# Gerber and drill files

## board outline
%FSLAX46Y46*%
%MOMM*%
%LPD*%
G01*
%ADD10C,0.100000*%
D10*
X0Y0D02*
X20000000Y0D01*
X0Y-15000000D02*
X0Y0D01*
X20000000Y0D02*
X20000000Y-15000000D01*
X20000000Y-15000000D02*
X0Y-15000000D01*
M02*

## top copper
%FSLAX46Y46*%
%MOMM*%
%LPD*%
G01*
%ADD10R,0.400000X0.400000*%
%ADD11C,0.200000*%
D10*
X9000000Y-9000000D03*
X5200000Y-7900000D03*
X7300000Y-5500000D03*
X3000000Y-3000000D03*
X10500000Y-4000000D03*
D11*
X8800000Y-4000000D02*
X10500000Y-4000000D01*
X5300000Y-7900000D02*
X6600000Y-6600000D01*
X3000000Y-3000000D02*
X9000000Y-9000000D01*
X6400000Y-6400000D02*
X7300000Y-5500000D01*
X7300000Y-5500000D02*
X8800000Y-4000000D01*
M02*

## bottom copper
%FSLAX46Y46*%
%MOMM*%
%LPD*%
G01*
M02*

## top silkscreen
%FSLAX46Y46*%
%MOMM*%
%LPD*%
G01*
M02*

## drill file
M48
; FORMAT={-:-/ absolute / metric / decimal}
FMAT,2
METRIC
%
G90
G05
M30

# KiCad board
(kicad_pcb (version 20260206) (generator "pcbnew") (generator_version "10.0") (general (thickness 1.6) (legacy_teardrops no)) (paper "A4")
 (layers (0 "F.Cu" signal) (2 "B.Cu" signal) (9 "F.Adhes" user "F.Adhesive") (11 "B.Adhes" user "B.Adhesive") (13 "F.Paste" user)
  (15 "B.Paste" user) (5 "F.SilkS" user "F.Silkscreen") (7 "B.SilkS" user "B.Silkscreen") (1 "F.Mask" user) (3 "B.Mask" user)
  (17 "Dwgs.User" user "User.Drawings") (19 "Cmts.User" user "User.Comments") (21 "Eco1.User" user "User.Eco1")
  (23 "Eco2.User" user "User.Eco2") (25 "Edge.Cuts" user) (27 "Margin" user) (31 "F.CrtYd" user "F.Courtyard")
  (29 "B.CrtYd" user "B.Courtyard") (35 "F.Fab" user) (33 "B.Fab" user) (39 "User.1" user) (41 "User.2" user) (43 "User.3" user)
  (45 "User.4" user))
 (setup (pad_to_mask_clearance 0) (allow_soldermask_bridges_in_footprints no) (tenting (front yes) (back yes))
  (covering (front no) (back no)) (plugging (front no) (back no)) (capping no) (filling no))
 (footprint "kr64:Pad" (layer "F.Cu") (at 9 9)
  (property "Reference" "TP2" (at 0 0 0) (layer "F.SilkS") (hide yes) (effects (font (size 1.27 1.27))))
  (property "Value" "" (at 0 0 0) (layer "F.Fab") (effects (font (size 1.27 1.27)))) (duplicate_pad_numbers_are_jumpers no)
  (pad "1" smd rect (at 0 0) (size 0.4 0.4) (layers "F.Cu" "F.Mask" "F.Paste") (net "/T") (thermal_bridge_angle 45)))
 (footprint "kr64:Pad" (layer "F.Cu") (at 5.2 7.9)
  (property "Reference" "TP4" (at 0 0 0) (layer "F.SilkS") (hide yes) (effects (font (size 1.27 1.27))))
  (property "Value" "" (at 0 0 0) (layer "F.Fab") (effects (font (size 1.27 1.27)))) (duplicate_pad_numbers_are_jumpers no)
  (pad "1" smd rect (at 0 0) (size 0.4 0.4) (layers "F.Cu" "F.Mask" "F.Paste") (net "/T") (thermal_bridge_angle 45)))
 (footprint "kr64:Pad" (layer "F.Cu") (at 7.3 5.5)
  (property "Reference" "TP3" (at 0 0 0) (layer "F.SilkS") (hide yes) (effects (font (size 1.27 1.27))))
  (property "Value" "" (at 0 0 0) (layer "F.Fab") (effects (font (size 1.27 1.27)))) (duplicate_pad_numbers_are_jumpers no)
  (pad "1" smd rect (at 0 0) (size 0.4 0.4) (layers "F.Cu" "F.Mask" "F.Paste") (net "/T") (thermal_bridge_angle 45)))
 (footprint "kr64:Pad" (layer "F.Cu") (at 3 3)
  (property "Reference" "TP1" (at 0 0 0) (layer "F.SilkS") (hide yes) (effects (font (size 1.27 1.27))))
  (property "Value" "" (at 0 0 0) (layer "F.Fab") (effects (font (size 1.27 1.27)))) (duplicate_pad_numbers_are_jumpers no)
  (pad "1" smd rect (at 0 0) (size 0.4 0.4) (layers "F.Cu" "F.Mask" "F.Paste") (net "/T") (thermal_bridge_angle 45)))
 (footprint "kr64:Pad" (layer "F.Cu") (at 10.5 4)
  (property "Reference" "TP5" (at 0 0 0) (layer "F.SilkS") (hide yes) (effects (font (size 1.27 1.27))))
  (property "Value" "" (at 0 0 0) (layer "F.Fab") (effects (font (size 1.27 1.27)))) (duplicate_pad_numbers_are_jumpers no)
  (pad "1" smd rect (at 0 0) (size 0.4 0.4) (layers "F.Cu" "F.Mask" "F.Paste") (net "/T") (thermal_bridge_angle 45)))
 (gr_line (start 0 0) (end 20 0) (stroke (width 0.1) (type default)) (layer "Edge.Cuts"))
 (gr_line (start 0 15) (end 0 0) (stroke (width 0.1) (type default)) (layer "Edge.Cuts"))
 (gr_line (start 20 0) (end 20 15) (stroke (width 0.1) (type default)) (layer "Edge.Cuts"))
 (gr_line (start 20 15) (end 0 15) (stroke (width 0.1) (type default)) (layer "Edge.Cuts"))
 (segment (start 8.8 4) (end 10.5 4) (width 0.2) (layer "F.Cu") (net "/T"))
 (segment (start 5.3 7.9) (end 6.6 6.6) (width 0.2) (layer "F.Cu") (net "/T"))
 (segment (start 3 3) (end 9 9) (width 0.2) (layer "F.Cu") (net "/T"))
 (segment (start 6.4 6.4) (end 7.3 5.5) (width 0.2) (layer "F.Cu") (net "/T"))
 (segment (start 7.3 5.5) (end 8.8 4) (width 0.2) (layer "F.Cu") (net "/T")))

